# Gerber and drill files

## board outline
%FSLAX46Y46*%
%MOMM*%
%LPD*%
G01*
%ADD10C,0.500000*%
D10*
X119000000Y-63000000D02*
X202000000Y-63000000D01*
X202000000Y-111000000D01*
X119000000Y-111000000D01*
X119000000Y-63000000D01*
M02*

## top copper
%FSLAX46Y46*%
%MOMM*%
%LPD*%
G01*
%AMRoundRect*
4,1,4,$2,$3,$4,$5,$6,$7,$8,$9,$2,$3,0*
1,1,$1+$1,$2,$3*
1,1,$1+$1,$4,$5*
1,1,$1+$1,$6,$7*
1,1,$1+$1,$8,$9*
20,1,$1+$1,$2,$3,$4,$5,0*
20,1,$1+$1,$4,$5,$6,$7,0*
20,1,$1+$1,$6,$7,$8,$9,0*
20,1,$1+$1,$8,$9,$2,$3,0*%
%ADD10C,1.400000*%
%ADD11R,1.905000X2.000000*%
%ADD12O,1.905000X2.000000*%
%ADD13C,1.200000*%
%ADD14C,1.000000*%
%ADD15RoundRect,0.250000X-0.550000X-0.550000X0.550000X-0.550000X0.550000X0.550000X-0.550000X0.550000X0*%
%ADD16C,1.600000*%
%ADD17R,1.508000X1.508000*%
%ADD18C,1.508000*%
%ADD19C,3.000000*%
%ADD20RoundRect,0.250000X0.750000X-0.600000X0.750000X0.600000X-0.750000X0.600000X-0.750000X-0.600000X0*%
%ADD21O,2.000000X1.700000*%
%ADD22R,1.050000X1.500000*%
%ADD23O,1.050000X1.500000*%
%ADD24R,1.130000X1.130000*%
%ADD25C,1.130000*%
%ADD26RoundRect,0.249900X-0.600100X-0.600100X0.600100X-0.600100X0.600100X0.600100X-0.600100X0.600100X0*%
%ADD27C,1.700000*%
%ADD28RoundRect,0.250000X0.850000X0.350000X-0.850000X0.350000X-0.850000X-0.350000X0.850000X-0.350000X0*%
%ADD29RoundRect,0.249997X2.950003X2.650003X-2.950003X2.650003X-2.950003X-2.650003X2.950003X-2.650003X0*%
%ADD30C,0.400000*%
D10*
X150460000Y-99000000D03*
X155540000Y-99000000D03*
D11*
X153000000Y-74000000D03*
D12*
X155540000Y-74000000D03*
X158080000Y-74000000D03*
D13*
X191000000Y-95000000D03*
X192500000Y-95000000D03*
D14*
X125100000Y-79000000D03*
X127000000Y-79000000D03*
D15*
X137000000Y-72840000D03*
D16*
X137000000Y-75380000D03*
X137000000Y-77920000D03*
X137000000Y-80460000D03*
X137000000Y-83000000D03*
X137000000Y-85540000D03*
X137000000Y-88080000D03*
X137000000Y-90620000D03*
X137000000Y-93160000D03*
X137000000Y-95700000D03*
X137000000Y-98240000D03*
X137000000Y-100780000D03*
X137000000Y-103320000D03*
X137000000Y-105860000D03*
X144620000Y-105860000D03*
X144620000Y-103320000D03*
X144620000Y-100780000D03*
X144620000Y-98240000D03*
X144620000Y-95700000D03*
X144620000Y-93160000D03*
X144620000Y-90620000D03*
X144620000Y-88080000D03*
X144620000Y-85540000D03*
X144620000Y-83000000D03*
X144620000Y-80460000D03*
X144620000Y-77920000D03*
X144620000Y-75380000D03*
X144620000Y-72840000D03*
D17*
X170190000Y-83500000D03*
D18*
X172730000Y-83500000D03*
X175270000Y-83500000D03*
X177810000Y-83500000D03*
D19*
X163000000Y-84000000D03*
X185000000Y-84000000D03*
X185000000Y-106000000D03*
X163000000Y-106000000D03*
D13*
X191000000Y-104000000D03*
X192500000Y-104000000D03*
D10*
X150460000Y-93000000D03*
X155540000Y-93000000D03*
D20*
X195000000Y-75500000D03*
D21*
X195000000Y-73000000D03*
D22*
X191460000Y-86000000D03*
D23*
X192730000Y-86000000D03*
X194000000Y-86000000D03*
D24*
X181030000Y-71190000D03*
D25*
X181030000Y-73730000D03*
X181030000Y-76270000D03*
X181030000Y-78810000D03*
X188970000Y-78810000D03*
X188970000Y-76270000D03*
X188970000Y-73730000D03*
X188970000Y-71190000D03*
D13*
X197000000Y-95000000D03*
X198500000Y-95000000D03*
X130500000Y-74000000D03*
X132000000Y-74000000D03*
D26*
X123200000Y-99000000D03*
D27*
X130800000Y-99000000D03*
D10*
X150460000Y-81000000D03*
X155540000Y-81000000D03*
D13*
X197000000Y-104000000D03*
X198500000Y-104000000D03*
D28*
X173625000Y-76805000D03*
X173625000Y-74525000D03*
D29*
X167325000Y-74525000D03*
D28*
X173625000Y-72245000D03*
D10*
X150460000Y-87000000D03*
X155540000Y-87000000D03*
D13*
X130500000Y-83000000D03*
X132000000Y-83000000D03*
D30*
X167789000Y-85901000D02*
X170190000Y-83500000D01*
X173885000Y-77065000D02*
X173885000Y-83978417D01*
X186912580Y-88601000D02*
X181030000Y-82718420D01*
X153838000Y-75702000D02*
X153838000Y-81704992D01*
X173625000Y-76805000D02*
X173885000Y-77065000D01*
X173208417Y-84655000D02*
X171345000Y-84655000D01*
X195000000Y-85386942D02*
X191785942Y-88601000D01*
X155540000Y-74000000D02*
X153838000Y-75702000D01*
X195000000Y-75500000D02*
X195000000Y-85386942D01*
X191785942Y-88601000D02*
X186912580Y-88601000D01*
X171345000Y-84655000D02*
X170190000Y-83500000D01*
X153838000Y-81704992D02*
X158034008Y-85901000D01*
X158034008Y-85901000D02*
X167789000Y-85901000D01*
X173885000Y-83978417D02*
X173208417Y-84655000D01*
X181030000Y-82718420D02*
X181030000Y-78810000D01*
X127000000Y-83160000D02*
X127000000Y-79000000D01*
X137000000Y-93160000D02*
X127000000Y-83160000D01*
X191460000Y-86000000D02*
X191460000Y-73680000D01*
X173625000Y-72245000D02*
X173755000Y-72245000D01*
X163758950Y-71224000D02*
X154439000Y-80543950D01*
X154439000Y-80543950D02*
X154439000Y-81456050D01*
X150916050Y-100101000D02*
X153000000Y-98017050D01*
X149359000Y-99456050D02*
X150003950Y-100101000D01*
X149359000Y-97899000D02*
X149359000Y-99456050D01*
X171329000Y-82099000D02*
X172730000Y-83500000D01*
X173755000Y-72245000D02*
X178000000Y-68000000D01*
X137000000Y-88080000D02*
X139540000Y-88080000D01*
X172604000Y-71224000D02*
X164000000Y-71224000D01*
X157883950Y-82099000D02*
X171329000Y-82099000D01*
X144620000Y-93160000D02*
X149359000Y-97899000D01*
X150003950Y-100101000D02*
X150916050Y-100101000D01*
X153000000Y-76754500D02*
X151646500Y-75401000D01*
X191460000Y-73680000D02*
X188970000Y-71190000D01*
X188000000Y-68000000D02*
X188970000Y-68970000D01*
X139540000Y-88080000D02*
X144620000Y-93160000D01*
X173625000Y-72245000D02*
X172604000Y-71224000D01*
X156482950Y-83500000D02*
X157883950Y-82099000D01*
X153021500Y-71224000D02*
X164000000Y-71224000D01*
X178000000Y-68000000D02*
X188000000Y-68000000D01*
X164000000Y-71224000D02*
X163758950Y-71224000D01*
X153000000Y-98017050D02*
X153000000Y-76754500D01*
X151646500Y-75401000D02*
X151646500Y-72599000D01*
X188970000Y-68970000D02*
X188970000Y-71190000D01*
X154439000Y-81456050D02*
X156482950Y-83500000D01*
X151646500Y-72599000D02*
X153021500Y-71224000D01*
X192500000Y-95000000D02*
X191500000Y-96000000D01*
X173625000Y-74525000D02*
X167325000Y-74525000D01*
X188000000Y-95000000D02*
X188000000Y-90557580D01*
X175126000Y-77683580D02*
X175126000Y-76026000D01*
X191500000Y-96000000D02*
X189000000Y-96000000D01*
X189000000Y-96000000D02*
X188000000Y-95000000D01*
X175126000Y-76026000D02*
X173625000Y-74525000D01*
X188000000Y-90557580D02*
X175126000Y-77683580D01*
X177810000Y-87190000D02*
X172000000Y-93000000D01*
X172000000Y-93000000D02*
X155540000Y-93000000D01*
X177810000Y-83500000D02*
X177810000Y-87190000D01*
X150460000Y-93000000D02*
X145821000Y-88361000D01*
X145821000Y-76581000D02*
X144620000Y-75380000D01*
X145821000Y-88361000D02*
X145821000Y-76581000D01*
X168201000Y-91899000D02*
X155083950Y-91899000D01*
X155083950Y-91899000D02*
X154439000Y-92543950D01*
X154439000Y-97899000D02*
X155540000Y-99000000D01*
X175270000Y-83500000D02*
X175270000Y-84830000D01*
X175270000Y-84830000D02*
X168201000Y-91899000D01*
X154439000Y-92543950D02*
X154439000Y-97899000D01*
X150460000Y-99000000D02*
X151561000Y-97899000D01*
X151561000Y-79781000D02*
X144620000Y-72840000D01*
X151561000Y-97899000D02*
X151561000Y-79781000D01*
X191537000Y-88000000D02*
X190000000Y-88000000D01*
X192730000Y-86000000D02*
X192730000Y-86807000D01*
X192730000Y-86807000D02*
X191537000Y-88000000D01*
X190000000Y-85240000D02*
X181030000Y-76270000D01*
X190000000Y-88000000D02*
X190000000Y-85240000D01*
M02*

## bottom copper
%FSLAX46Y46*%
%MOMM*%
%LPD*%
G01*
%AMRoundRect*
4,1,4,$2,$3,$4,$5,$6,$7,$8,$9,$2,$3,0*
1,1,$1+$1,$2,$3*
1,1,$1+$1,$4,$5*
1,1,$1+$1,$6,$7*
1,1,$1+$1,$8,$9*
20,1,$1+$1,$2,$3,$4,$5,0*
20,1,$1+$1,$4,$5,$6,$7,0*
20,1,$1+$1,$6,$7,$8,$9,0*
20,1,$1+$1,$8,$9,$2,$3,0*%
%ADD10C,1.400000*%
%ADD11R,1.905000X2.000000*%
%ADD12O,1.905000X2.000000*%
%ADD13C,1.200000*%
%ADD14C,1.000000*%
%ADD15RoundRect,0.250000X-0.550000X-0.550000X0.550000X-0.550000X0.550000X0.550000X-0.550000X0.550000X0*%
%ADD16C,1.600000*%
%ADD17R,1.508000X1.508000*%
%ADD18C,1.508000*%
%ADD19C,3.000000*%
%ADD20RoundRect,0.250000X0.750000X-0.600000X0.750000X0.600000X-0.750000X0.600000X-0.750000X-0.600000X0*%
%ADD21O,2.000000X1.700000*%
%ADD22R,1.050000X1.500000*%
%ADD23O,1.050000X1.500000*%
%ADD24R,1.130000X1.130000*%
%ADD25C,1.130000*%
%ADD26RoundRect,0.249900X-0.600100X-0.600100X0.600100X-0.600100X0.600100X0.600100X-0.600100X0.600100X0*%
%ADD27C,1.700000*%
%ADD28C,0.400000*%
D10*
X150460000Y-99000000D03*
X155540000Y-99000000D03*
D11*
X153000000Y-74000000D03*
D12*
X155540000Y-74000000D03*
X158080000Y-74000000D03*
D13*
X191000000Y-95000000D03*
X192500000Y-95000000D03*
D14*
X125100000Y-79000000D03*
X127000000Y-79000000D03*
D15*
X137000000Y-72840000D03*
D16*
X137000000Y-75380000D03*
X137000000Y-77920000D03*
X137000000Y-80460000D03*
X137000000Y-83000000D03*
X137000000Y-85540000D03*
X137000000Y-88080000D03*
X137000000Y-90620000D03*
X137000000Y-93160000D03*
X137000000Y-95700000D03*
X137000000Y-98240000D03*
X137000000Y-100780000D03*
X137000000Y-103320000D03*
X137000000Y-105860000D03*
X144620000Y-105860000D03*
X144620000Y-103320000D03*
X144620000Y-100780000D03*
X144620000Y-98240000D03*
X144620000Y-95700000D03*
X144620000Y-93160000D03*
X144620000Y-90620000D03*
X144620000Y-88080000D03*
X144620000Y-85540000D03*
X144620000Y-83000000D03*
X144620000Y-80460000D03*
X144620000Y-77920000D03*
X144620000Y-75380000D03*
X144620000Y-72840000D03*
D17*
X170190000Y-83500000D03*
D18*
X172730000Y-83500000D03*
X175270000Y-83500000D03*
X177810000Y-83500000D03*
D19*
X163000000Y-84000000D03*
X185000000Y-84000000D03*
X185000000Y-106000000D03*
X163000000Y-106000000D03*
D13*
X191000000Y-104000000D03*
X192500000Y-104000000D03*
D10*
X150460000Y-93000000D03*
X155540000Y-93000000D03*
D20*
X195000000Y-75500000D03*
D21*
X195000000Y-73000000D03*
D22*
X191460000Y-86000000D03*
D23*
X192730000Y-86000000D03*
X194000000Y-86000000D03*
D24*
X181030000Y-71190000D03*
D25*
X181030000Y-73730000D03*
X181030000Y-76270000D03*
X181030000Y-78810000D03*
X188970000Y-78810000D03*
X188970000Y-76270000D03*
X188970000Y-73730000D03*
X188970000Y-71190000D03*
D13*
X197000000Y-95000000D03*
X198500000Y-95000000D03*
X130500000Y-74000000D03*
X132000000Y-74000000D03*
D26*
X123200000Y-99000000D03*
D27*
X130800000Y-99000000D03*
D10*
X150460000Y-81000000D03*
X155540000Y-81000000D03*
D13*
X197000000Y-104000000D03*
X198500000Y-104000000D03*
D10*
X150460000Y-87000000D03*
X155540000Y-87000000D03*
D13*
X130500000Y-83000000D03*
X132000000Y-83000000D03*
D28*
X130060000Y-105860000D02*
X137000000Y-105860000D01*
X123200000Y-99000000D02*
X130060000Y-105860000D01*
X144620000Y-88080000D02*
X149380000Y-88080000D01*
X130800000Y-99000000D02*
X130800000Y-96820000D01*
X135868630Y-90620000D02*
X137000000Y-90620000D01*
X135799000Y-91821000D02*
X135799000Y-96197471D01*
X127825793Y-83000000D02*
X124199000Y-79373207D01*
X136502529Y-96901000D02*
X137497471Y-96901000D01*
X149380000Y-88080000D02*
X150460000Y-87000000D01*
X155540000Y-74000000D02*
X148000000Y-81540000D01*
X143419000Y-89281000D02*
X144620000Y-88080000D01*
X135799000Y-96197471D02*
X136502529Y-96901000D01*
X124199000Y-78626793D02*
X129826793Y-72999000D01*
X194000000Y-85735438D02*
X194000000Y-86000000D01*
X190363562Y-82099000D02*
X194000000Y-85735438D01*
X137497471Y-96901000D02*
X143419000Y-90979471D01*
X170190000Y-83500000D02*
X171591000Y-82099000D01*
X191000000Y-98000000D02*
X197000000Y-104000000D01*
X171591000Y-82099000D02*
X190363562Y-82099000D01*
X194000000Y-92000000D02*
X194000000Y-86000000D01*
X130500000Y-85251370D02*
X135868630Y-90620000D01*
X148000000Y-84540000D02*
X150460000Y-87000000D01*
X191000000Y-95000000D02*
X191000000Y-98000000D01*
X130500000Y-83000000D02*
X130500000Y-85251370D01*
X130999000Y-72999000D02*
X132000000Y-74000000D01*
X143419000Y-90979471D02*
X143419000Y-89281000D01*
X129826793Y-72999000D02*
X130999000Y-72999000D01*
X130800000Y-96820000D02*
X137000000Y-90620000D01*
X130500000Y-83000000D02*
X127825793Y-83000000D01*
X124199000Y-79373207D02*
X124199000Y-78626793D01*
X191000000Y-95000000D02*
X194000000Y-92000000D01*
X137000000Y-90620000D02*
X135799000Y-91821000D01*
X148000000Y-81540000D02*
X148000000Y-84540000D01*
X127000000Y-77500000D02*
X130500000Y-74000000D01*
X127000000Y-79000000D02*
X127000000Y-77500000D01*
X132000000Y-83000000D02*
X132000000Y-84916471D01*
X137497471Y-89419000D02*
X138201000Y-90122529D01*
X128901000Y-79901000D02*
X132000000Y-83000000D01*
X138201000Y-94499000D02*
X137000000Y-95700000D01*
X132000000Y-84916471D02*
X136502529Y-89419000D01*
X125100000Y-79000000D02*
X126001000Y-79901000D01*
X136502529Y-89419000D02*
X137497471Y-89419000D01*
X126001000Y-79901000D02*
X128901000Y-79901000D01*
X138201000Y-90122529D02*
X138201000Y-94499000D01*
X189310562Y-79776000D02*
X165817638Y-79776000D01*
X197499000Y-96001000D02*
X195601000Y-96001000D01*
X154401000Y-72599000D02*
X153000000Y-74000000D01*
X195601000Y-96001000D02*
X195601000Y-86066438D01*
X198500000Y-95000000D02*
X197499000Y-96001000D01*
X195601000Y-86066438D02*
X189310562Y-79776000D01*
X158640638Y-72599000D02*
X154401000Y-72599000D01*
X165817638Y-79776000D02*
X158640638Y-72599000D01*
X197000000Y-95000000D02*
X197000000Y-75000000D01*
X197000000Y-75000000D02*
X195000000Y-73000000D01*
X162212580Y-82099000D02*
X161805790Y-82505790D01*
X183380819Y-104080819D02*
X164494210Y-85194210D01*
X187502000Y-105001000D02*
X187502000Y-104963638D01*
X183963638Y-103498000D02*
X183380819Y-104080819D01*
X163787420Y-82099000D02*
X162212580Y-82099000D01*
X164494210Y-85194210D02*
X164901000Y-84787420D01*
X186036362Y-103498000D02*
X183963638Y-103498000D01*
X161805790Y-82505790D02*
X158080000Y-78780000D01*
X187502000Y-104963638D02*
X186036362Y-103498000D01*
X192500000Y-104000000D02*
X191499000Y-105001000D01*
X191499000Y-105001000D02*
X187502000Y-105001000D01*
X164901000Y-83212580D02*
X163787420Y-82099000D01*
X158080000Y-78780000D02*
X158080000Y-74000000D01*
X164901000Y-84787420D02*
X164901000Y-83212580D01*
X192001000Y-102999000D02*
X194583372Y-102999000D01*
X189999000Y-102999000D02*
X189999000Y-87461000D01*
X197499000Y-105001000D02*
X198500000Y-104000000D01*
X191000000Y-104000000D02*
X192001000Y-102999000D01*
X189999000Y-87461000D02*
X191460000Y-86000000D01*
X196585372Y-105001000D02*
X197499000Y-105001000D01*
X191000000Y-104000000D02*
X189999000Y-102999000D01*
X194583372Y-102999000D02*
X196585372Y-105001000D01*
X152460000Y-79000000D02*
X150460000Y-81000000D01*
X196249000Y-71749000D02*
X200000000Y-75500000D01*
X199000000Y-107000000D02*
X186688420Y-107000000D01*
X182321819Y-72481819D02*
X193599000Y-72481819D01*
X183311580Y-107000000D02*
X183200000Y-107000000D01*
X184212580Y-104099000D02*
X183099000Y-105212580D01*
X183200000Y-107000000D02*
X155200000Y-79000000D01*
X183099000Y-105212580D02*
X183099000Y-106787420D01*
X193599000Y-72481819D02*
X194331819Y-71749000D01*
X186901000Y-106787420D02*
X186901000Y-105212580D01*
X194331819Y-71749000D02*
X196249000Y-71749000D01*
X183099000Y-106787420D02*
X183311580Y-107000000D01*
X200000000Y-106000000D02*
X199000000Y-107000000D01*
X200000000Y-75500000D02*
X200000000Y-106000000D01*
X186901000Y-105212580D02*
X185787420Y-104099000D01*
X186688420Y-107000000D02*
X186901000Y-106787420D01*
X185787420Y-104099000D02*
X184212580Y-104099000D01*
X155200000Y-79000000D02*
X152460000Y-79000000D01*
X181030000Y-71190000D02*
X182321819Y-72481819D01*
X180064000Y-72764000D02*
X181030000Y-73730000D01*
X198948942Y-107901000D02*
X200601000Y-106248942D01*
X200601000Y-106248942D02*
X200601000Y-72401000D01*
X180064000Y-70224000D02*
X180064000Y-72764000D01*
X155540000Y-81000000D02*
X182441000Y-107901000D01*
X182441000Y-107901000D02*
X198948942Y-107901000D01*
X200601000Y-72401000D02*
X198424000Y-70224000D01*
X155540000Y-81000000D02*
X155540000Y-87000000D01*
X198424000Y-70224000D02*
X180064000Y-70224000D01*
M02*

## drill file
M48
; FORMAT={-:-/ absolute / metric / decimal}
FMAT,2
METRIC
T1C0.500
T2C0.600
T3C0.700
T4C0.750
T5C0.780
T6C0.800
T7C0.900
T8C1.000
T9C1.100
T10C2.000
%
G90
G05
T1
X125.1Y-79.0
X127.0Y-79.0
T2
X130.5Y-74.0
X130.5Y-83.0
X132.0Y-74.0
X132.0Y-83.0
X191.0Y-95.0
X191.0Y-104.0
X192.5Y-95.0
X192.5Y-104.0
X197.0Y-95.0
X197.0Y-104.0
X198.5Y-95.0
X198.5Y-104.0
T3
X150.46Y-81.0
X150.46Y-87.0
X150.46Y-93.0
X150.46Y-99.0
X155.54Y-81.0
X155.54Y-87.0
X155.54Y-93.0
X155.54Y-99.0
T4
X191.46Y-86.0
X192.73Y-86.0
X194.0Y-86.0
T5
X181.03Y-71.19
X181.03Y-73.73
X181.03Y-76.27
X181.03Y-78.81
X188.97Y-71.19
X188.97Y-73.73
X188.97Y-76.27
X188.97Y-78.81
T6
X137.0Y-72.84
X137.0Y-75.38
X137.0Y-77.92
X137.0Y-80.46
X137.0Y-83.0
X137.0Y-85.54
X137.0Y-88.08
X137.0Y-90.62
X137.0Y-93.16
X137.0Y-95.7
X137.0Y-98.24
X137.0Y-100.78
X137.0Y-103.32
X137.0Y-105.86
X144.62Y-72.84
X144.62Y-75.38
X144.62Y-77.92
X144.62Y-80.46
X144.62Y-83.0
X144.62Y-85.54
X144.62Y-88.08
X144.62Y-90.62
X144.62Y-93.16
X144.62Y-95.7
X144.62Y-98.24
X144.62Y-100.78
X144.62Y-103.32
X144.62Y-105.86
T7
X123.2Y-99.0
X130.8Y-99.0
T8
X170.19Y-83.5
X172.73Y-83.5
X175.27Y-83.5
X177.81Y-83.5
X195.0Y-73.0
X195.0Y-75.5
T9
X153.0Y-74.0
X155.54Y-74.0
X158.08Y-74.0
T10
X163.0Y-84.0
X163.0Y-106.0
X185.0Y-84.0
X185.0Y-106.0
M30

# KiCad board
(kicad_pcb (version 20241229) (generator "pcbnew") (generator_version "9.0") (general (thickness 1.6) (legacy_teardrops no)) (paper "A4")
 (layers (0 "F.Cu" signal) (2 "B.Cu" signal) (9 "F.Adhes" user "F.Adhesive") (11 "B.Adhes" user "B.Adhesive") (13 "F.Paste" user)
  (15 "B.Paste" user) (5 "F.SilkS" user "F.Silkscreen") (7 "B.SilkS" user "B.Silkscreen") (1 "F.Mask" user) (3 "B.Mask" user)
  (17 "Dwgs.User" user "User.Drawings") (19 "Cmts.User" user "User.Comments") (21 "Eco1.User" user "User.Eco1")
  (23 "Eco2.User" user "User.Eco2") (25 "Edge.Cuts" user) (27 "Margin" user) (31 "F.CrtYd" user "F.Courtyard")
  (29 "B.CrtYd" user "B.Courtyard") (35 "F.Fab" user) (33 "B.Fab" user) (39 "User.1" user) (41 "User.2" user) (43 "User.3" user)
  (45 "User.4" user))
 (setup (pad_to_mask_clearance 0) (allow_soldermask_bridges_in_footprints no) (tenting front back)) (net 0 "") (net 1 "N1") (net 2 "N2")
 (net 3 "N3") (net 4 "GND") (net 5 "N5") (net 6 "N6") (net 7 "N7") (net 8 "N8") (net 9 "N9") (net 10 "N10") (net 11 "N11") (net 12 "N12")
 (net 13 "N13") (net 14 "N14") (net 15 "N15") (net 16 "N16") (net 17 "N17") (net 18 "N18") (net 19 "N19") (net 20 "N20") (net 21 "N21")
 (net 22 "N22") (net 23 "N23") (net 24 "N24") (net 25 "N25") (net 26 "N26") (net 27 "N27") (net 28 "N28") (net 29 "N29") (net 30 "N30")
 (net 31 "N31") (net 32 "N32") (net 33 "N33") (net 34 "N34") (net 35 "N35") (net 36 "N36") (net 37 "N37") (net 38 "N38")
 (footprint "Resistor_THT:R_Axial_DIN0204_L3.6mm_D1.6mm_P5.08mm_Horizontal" (layer "F.Cu") (at 150.46 99)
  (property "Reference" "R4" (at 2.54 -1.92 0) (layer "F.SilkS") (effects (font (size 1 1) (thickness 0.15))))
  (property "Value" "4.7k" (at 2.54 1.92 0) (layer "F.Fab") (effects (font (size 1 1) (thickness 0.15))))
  (pad "1" thru_hole circle (at 0 0) (size 1.4 1.4) (drill 0.7) (layers "*.Cu" "*.Mask") (remove_unused_layers no) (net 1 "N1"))
  (pad "2" thru_hole circle (at 5.08 0) (size 1.4 1.4) (drill 0.7) (layers "*.Cu" "*.Mask") (remove_unused_layers no) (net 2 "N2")))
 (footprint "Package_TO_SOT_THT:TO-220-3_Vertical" (layer "F.Cu") (at 153 74)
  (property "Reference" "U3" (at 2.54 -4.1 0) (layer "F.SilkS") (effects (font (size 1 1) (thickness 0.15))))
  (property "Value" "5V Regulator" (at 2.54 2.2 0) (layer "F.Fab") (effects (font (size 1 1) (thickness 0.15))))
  (pad "1" thru_hole rect (at 0 0) (size 1.905 2) (drill 1.1) (layers "*.Cu" "*.Mask") (remove_unused_layers no) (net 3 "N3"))
  (pad "2" thru_hole oval (at 2.54 0) (size 1.905 2) (drill 1.1) (layers "*.Cu" "*.Mask") (remove_unused_layers no) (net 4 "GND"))
  (pad "3" thru_hole oval (at 5.08 0) (size 1.905 2) (drill 1.1) (layers "*.Cu" "*.Mask") (remove_unused_layers no) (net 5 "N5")))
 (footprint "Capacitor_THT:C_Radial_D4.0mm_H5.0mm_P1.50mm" (layer "F.Cu") (at 191 95)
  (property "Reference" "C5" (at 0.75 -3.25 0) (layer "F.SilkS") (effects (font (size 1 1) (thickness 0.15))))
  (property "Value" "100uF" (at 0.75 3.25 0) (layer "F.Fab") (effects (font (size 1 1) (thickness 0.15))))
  (pad "1" thru_hole circle (at 0 0) (size 1.2 1.2) (drill 0.6) (layers "*.Cu" "*.Mask") (remove_unused_layers no) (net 4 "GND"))
  (pad "2" thru_hole circle (at 1.5 0) (size 1.2 1.2) (drill 0.6) (layers "*.Cu" "*.Mask") (remove_unused_layers no) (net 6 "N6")))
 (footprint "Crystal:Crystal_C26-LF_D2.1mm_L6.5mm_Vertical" (layer "F.Cu") (at 125.1 79)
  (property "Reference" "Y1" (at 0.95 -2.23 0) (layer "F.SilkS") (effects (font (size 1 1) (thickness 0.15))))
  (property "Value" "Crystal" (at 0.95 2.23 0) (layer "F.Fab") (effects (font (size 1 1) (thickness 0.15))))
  (pad "1" thru_hole circle (at 0 0) (size 1 1) (drill 0.5) (layers "*.Cu" "*.Mask") (remove_unused_layers no) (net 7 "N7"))
  (pad "2" thru_hole circle (at 1.9 0) (size 1 1) (drill 0.5) (layers "*.Cu" "*.Mask") (remove_unused_layers no) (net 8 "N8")))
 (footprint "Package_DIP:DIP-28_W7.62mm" (layer "F.Cu") (at 137 72.84)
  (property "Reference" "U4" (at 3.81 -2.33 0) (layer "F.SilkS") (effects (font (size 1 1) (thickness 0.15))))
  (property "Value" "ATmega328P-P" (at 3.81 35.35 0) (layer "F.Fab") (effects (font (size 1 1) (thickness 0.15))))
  (pad "1" thru_hole roundrect (at 0 0) (size 1.6 1.6) (drill 0.8) (layers "*.Cu" "*.Mask") (remove_unused_layers no)
   (roundrect_rratio 0.15625) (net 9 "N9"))
  (pad "2" thru_hole circle (at 0 2.54) (size 1.6 1.6) (drill 0.8) (layers "*.Cu" "*.Mask") (remove_unused_layers no) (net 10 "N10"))
  (pad "3" thru_hole circle (at 0 5.08) (size 1.6 1.6) (drill 0.8) (layers "*.Cu" "*.Mask") (remove_unused_layers no) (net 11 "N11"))
  (pad "4" thru_hole circle (at 0 7.62) (size 1.6 1.6) (drill 0.8) (layers "*.Cu" "*.Mask") (remove_unused_layers no) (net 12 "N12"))
  (pad "5" thru_hole circle (at 0 10.16) (size 1.6 1.6) (drill 0.8) (layers "*.Cu" "*.Mask") (remove_unused_layers no) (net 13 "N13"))
  (pad "6" thru_hole circle (at 0 12.7) (size 1.6 1.6) (drill 0.8) (layers "*.Cu" "*.Mask") (remove_unused_layers no) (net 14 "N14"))
  (pad "7" thru_hole circle (at 0 15.24) (size 1.6 1.6) (drill 0.8) (layers "*.Cu" "*.Mask") (remove_unused_layers no) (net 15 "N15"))
  (pad "8" thru_hole circle (at 0 17.78) (size 1.6 1.6) (drill 0.8) (layers "*.Cu" "*.Mask") (remove_unused_layers no) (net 4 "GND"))
  (pad "9" thru_hole circle (at 0 20.32) (size 1.6 1.6) (drill 0.8) (layers "*.Cu" "*.Mask") (remove_unused_layers no) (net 8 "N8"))
  (pad "10" thru_hole circle (at 0 22.86) (size 1.6 1.6) (drill 0.8) (layers "*.Cu" "*.Mask") (remove_unused_layers no) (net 7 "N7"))
  (pad "11" thru_hole circle (at 0 25.4) (size 1.6 1.6) (drill 0.8) (layers "*.Cu" "*.Mask") (remove_unused_layers no) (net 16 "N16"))
  (pad "12" thru_hole circle (at 0 27.94) (size 1.6 1.6) (drill 0.8) (layers "*.Cu" "*.Mask") (remove_unused_layers no) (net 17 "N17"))
  (pad "13" thru_hole circle (at 0 30.48) (size 1.6 1.6) (drill 0.8) (layers "*.Cu" "*.Mask") (remove_unused_layers no) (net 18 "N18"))
  (pad "14" thru_hole circle (at 0 33.02) (size 1.6 1.6) (drill 0.8) (layers "*.Cu" "*.Mask") (remove_unused_layers no) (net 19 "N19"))
  (pad "15" thru_hole circle (at 7.62 33.02) (size 1.6 1.6) (drill 0.8) (layers "*.Cu" "*.Mask") (remove_unused_layers no) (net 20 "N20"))
  (pad "16" thru_hole circle (at 7.62 30.48) (size 1.6 1.6) (drill 0.8) (layers "*.Cu" "*.Mask") (remove_unused_layers no) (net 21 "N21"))
  (pad "17" thru_hole circle (at 7.62 27.94) (size 1.6 1.6) (drill 0.8) (layers "*.Cu" "*.Mask") (remove_unused_layers no) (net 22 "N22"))
  (pad "18" thru_hole circle (at 7.62 25.4) (size 1.6 1.6) (drill 0.8) (layers "*.Cu" "*.Mask") (remove_unused_layers no) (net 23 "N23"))
  (pad "19" thru_hole circle (at 7.62 22.86) (size 1.6 1.6) (drill 0.8) (layers "*.Cu" "*.Mask") (remove_unused_layers no) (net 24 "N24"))
  (pad "20" thru_hole circle (at 7.62 20.32) (size 1.6 1.6) (drill 0.8) (layers "*.Cu" "*.Mask") (remove_unused_layers no) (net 15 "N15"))
  (pad "21" thru_hole circle (at 7.62 17.78) (size 1.6 1.6) (drill 0.8) (layers "*.Cu" "*.Mask") (remove_unused_layers no) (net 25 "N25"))
  (pad "22" thru_hole circle (at 7.62 15.24) (size 1.6 1.6) (drill 0.8) (layers "*.Cu" "*.Mask") (remove_unused_layers no) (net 4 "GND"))
  (pad "23" thru_hole circle (at 7.62 12.7) (size 1.6 1.6) (drill 0.8) (layers "*.Cu" "*.Mask") (remove_unused_layers no) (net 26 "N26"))
  (pad "24" thru_hole circle (at 7.62 10.16) (size 1.6 1.6) (drill 0.8) (layers "*.Cu" "*.Mask") (remove_unused_layers no) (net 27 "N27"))
  (pad "25" thru_hole circle (at 7.62 7.62) (size 1.6 1.6) (drill 0.8) (layers "*.Cu" "*.Mask") (remove_unused_layers no) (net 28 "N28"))
  (pad "26" thru_hole circle (at 7.62 5.08) (size 1.6 1.6) (drill 0.8) (layers "*.Cu" "*.Mask") (remove_unused_layers no) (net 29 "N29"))
  (pad "27" thru_hole circle (at 7.62 2.54) (size 1.6 1.6) (drill 0.8) (layers "*.Cu" "*.Mask") (remove_unused_layers no) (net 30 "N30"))
  (pad "28" thru_hole circle (at 7.62 0) (size 1.6 1.6) (drill 0.8) (layers "*.Cu" "*.Mask") (remove_unused_layers no) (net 1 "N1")))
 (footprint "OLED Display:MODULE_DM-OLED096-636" (layer "F.Cu") (at 174 95)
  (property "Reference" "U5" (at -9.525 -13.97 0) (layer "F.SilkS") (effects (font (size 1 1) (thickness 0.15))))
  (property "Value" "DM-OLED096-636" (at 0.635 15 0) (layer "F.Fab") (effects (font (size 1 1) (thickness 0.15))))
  (pad "1" thru_hole rect (at -3.81 -11.5) (size 1.508 1.508) (drill 1) (layers "*.Cu" "*.Mask") (remove_unused_layers no) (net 4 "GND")
   (solder_mask_margin 0.102))
  (pad "2" thru_hole circle (at -1.27 -11.5) (size 1.508 1.508) (drill 1) (layers "*.Cu" "*.Mask") (remove_unused_layers no) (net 15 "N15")
   (solder_mask_margin 0.102))
  (pad "3" thru_hole circle (at 1.27 -11.5) (size 1.508 1.508) (drill 1) (layers "*.Cu" "*.Mask") (remove_unused_layers no) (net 2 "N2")
   (solder_mask_margin 0.102))
  (pad "4" thru_hole circle (at 3.81 -11.5) (size 1.508 1.508) (drill 1) (layers "*.Cu" "*.Mask") (remove_unused_layers no) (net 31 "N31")
   (solder_mask_margin 0.102))
  (pad "S1" thru_hole circle (at -11 -11) (size 3 3) (drill 2) (layers "*.Cu" "*.Mask") (remove_unused_layers no) (solder_mask_margin 0.102))
  (pad "S2" thru_hole circle (at 11 -11) (size 3 3) (drill 2) (layers "*.Cu" "*.Mask") (remove_unused_layers no) (solder_mask_margin 0.102))
  (pad "S3" thru_hole circle (at 11 11) (size 3 3) (drill 2) (layers "*.Cu" "*.Mask") (remove_unused_layers no) (solder_mask_margin 0.102))
  (pad "S4" thru_hole circle (at -11 11) (size 3 3) (drill 2) (layers "*.Cu" "*.Mask") (remove_unused_layers no) (solder_mask_margin 0.102)))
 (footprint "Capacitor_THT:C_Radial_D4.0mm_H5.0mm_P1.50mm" (layer "F.Cu") (at 191 104)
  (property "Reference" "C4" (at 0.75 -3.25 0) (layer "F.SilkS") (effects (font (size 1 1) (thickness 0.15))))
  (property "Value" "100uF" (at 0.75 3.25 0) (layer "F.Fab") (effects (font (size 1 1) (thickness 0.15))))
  (pad "1" thru_hole circle (at 0 0) (size 1.2 1.2) (drill 0.6) (layers "*.Cu" "*.Mask") (remove_unused_layers no) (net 15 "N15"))
  (pad "2" thru_hole circle (at 1.5 0) (size 1.2 1.2) (drill 0.6) (layers "*.Cu" "*.Mask") (remove_unused_layers no) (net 5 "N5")))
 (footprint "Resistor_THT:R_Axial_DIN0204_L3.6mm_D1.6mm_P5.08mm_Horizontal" (layer "F.Cu") (at 150.46 93)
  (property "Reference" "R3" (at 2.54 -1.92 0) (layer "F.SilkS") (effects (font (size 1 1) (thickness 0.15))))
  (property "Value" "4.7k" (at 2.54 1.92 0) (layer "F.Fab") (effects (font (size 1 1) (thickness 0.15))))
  (pad "1" thru_hole circle (at 0 0) (size 1.4 1.4) (drill 0.7) (layers "*.Cu" "*.Mask") (remove_unused_layers no) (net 30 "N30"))
  (pad "2" thru_hole circle (at 5.08 0) (size 1.4 1.4) (drill 0.7) (layers "*.Cu" "*.Mask") (remove_unused_layers no) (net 31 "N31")))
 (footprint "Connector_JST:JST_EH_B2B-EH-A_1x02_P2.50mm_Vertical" (layer "F.Cu") (at 195 75.5 90)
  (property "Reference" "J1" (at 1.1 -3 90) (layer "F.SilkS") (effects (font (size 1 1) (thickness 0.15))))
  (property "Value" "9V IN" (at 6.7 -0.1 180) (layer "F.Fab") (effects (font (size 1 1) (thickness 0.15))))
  (pad "1" thru_hole roundrect (at 0 0 90) (size 1.7 2) (drill 1) (layers "*.Cu" "*.Mask") (remove_unused_layers no)
   (roundrect_rratio 0.147059) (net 4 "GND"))
  (pad "2" thru_hole oval (at 2.5 0 90) (size 1.7 2) (drill 1) (layers "*.Cu" "*.Mask") (remove_unused_layers no) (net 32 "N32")))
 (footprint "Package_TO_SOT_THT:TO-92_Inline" (layer "F.Cu") (at 191.46 86)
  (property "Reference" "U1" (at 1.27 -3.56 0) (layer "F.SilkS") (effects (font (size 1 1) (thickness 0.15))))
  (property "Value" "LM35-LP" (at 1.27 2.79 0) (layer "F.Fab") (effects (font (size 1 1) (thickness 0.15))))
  (pad "1" thru_hole rect (at 0 0) (size 1.05 1.5) (drill 0.75) (layers "*.Cu" "*.Mask") (remove_unused_layers no) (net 15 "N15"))
  (pad "2" thru_hole oval (at 1.27 0) (size 1.05 1.5) (drill 0.75) (layers "*.Cu" "*.Mask") (remove_unused_layers no) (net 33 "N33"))
  (pad "3" thru_hole oval (at 2.54 0) (size 1.05 1.5) (drill 0.75) (layers "*.Cu" "*.Mask") (remove_unused_layers no) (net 4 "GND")))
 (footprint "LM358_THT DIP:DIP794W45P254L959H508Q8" (layer "F.Cu") (at 185 75)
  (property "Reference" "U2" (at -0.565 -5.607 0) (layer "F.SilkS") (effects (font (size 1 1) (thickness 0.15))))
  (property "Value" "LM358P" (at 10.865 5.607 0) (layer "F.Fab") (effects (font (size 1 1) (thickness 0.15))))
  (pad "1" thru_hole rect (at -3.97 -3.81) (size 1.13 1.13) (drill 0.78) (layers "*.Cu" "*.Mask") (remove_unused_layers no) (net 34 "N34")
   (solder_mask_margin 0.102))
  (pad "2" thru_hole circle (at -3.97 -1.27) (size 1.13 1.13) (drill 0.78) (layers "*.Cu" "*.Mask") (remove_unused_layers no) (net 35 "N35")
   (solder_mask_margin 0.102))
  (pad "3" thru_hole circle (at -3.97 1.27) (size 1.13 1.13) (drill 0.78) (layers "*.Cu" "*.Mask") (remove_unused_layers no) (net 33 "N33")
   (solder_mask_margin 0.102))
  (pad "4" thru_hole circle (at -3.97 3.81) (size 1.13 1.13) (drill 0.78) (layers "*.Cu" "*.Mask") (remove_unused_layers no) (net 4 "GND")
   (solder_mask_margin 0.102))
  (pad "5" thru_hole circle (at 3.97 3.81) (size 1.13 1.13) (drill 0.78) (layers "*.Cu" "*.Mask") (remove_unused_layers no) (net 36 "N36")
   (solder_mask_margin 0.102))
  (pad "6" thru_hole circle (at 3.97 1.27) (size 1.13 1.13) (drill 0.78) (layers "*.Cu" "*.Mask") (remove_unused_layers no) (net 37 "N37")
   (solder_mask_margin 0.102))
  (pad "7" thru_hole circle (at 3.97 -1.27) (size 1.13 1.13) (drill 0.78) (layers "*.Cu" "*.Mask") (remove_unused_layers no) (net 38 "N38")
   (solder_mask_margin 0.102))
  (pad "8" thru_hole circle (at 3.97 -3.81) (size 1.13 1.13) (drill 0.78) (layers "*.Cu" "*.Mask") (remove_unused_layers no) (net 15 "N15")
   (solder_mask_margin 0.102)))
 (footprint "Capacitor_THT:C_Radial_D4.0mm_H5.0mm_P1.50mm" (layer "F.Cu") (at 197 95)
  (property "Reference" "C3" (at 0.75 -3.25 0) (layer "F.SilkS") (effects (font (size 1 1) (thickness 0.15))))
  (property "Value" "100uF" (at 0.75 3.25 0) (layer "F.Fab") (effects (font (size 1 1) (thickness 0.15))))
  (pad "1" thru_hole circle (at 0 0) (size 1.2 1.2) (drill 0.6) (layers "*.Cu" "*.Mask") (remove_unused_layers no) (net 32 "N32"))
  (pad "2" thru_hole circle (at 1.5 0) (size 1.2 1.2) (drill 0.6) (layers "*.Cu" "*.Mask") (remove_unused_layers no) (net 3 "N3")))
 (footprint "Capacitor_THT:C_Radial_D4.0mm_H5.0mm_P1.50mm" (layer "F.Cu") (at 130.5 74)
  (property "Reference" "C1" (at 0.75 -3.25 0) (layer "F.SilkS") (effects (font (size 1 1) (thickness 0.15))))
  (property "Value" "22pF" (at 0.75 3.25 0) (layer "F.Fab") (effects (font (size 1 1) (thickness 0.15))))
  (pad "1" thru_hole circle (at 0 0) (size 1.2 1.2) (drill 0.6) (layers "*.Cu" "*.Mask") (remove_unused_layers no) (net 8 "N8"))
  (pad "2" thru_hole circle (at 1.5 0) (size 1.2 1.2) (drill 0.6) (layers "*.Cu" "*.Mask") (remove_unused_layers no) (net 4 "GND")))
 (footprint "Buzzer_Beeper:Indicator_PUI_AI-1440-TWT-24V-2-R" (layer "F.Cu") (at 123.2 99)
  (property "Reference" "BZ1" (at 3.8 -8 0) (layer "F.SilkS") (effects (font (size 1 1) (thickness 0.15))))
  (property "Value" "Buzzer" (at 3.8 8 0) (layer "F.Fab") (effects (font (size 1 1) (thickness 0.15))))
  (pad "1" thru_hole roundrect (at 0 0) (size 1.7 1.7) (drill 0.9) (layers "*.Cu" "*.Mask") (remove_unused_layers no)
   (roundrect_rratio 0.147) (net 19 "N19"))
  (pad "2" thru_hole circle (at 7.6 0) (size 1.7 1.7) (drill 0.9) (layers "*.Cu" "*.Mask") (remove_unused_layers no) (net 4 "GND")))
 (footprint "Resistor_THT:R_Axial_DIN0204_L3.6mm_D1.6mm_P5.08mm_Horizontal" (layer "F.Cu") (at 150.46 81)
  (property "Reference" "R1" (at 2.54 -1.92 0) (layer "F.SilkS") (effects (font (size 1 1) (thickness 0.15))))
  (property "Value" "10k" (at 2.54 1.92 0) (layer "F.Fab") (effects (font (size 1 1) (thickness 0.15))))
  (pad "1" thru_hole circle (at 0 0) (size 1.4 1.4) (drill 0.7) (layers "*.Cu" "*.Mask") (remove_unused_layers no) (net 34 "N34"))
  (pad "2" thru_hole circle (at 5.08 0) (size 1.4 1.4) (drill 0.7) (layers "*.Cu" "*.Mask") (remove_unused_layers no) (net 35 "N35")))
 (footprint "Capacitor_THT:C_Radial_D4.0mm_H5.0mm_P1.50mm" (layer "F.Cu") (at 197 104)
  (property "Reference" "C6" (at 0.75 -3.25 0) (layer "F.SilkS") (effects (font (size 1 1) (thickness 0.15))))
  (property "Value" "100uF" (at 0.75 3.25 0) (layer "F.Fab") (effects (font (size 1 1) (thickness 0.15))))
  (pad "1" thru_hole circle (at 0 0) (size 1.2 1.2) (drill 0.6) (layers "*.Cu" "*.Mask") (remove_unused_layers no) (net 4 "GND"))
  (pad "2" thru_hole circle (at 1.5 0) (size 1.2 1.2) (drill 0.6) (layers "*.Cu" "*.Mask") (remove_unused_layers no) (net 15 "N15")))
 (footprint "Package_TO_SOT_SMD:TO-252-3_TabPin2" (layer "F.Cu") (at 168.585 74.525 180)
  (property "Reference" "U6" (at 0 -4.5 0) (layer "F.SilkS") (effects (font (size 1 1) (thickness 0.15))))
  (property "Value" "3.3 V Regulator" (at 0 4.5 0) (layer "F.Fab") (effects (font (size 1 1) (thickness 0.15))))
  (pad "" smd roundrect (at -0.415 -1.525 180) (size 3.05 2.75) (layers "F.Paste") (roundrect_rratio 0.090909))
  (pad "" smd roundrect (at -0.415 1.525 180) (size 3.05 2.75) (layers "F.Paste") (roundrect_rratio 0.090909))
  (pad "" smd roundrect (at 2.935 -1.525 180) (size 3.05 2.75) (layers "F.Paste") (roundrect_rratio 0.090909))
  (pad "" smd roundrect (at 2.935 1.525 180) (size 3.05 2.75) (layers "F.Paste") (roundrect_rratio 0.090909))
  (pad "1" smd roundrect (at -5.04 -2.28 180) (size 2.2 1.2) (layers "F.Cu" "F.Mask" "F.Paste") (roundrect_rratio 0.208333) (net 4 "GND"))
  (pad "2" smd roundrect (at -5.04 0 180) (size 2.2 1.2) (layers "F.Cu" "F.Mask" "F.Paste") (roundrect_rratio 0.208333) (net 6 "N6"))
  (pad "2" smd roundrect (at 1.26 0 180) (size 6.4 5.8) (layers "F.Cu" "F.Mask") (roundrect_rratio 0.043103) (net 6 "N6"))
  (pad "3" smd roundrect (at -5.04 2.28 180) (size 2.2 1.2) (layers "F.Cu" "F.Mask" "F.Paste") (roundrect_rratio 0.208333) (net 15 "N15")))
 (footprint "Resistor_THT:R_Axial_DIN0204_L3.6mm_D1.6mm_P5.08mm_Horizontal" (layer "F.Cu") (at 150.46 87)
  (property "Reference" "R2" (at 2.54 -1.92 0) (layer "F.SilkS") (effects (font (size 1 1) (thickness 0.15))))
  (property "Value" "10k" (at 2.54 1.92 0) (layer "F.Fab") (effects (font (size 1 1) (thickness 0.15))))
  (pad "1" thru_hole circle (at 0 0) (size 1.4 1.4) (drill 0.7) (layers "*.Cu" "*.Mask") (remove_unused_layers no) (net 4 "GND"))
  (pad "2" thru_hole circle (at 5.08 0) (size 1.4 1.4) (drill 0.7) (layers "*.Cu" "*.Mask") (remove_unused_layers no) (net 35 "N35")))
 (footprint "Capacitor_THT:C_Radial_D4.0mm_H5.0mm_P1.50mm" (layer "F.Cu") (at 130.5 83)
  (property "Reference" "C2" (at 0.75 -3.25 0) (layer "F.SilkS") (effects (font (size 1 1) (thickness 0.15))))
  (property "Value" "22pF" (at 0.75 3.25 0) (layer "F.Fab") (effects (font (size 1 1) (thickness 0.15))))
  (pad "1" thru_hole circle (at 0 0) (size 1.2 1.2) (drill 0.6) (layers "*.Cu" "*.Mask") (remove_unused_layers no) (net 4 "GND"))
  (pad "2" thru_hole circle (at 1.5 0) (size 1.2 1.2) (drill 0.6) (layers "*.Cu" "*.Mask") (remove_unused_layers no) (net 7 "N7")))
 (gr_rect (start 119 63) (end 202 111) (stroke (width 0.5) (type solid)) (fill no) (layer "Edge.Cuts"))
 (segment (start 130.06 105.86) (end 137 105.86) (width 0.4) (layer "B.Cu") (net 19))
 (segment (start 123.2 99) (end 130.06 105.86) (width 0.4) (layer "B.Cu") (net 19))
 (segment (start 167.789 85.901) (end 170.19 83.5) (width 0.4) (layer "F.Cu") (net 4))
 (segment (start 173.885 77.065) (end 173.885 83.978417) (width 0.4) (layer "F.Cu") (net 4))
 (segment (start 186.91258 88.601) (end 181.03 82.71842) (width 0.4) (layer "F.Cu") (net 4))
 (segment (start 153.838 75.702) (end 153.838 81.704992) (width 0.4) (layer "F.Cu") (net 4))
 (segment (start 173.625 76.805) (end 173.885 77.065) (width 0.4) (layer "F.Cu") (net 4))
 (segment (start 173.208417 84.655) (end 171.345 84.655) (width 0.4) (layer "F.Cu") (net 4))
 (segment (start 195 85.386942) (end 191.785942 88.601) (width 0.4) (layer "F.Cu") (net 4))
 (segment (start 155.54 74) (end 153.838 75.702) (width 0.4) (layer "F.Cu") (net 4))
 (segment (start 195 75.5) (end 195 85.386942) (width 0.4) (layer "F.Cu") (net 4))
 (segment (start 191.785942 88.601) (end 186.91258 88.601) (width 0.4) (layer "F.Cu") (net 4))
 (segment (start 171.345 84.655) (end 170.19 83.5) (width 0.4) (layer "F.Cu") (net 4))
 (segment (start 153.838 81.704992) (end 158.034008 85.901) (width 0.4) (layer "F.Cu") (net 4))
 (segment (start 158.034008 85.901) (end 167.789 85.901) (width 0.4) (layer "F.Cu") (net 4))
 (segment (start 173.885 83.978417) (end 173.208417 84.655) (width 0.4) (layer "F.Cu") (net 4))
 (segment (start 181.03 82.71842) (end 181.03 78.81) (width 0.4) (layer "F.Cu") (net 4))
 (segment (start 144.62 88.08) (end 149.38 88.08) (width 0.4) (layer "B.Cu") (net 4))
 (segment (start 130.8 99) (end 130.8 96.82) (width 0.4) (layer "B.Cu") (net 4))
 (segment (start 135.86863 90.62) (end 137 90.62) (width 0.4) (layer "B.Cu") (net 4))
 (segment (start 135.799 91.821) (end 135.799 96.197471) (width 0.4) (layer "B.Cu") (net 4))
 (segment (start 127.825793 83) (end 124.199 79.373207) (width 0.4) (layer "B.Cu") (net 4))
 (segment (start 136.502529 96.901) (end 137.497471 96.901) (width 0.4) (layer "B.Cu") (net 4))
 (segment (start 149.38 88.08) (end 150.46 87) (width 0.4) (layer "B.Cu") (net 4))
 (segment (start 155.54 74) (end 148 81.54) (width 0.4) (layer "B.Cu") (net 4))
 (segment (start 143.419 89.281) (end 144.62 88.08) (width 0.4) (layer "B.Cu") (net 4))
 (segment (start 135.799 96.197471) (end 136.502529 96.901) (width 0.4) (layer "B.Cu") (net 4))
 (segment (start 124.199 78.626793) (end 129.826793 72.999) (width 0.4) (layer "B.Cu") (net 4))
 (segment (start 194 85.735438) (end 194 86) (width 0.4) (layer "B.Cu") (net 4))
 (segment (start 190.363562 82.099) (end 194 85.735438) (width 0.4) (layer "B.Cu") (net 4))
 (segment (start 137.497471 96.901) (end 143.419 90.979471) (width 0.4) (layer "B.Cu") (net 4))
 (segment (start 170.19 83.5) (end 171.591 82.099) (width 0.4) (layer "B.Cu") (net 4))
 (segment (start 191 98) (end 197 104) (width 0.4) (layer "B.Cu") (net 4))
 (segment (start 171.591 82.099) (end 190.363562 82.099) (width 0.4) (layer "B.Cu") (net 4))
 (segment (start 194 92) (end 194 86) (width 0.4) (layer "B.Cu") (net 4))
 (segment (start 130.5 85.25137) (end 135.86863 90.62) (width 0.4) (layer "B.Cu") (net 4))
 (segment (start 148 84.54) (end 150.46 87) (width 0.4) (layer "B.Cu") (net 4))
 (segment (start 191 95) (end 191 98) (width 0.4) (layer "B.Cu") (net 4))
 (segment (start 130.5 83) (end 130.5 85.25137) (width 0.4) (layer "B.Cu") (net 4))
 (segment (start 130.999 72.999) (end 132 74) (width 0.4) (layer "B.Cu") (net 4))
 (segment (start 143.419 90.979471) (end 143.419 89.281) (width 0.4) (layer "B.Cu") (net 4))
 (segment (start 129.826793 72.999) (end 130.999 72.999) (width 0.4) (layer "B.Cu") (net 4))
 (segment (start 130.8 96.82) (end 137 90.62) (width 0.4) (layer "B.Cu") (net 4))
 (segment (start 130.5 83) (end 127.825793 83) (width 0.4) (layer "B.Cu") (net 4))
 (segment (start 124.199 79.373207) (end 124.199 78.626793) (width 0.4) (layer "B.Cu") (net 4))
 (segment (start 191 95) (end 194 92) (width 0.4) (layer "B.Cu") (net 4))
 (segment (start 137 90.62) (end 135.799 91.821) (width 0.4) (layer "B.Cu") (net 4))
 (segment (start 148 81.54) (end 148 84.54) (width 0.4) (layer "B.Cu") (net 4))
 (segment (start 127 83.16) (end 127 79) (width 0.4) (layer "F.Cu") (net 8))
 (segment (start 137 93.16) (end 127 83.16) (width 0.4) (layer "F.Cu") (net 8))
 (segment (start 127 77.5) (end 130.5 74) (width 0.4) (layer "B.Cu") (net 8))
 (segment (start 127 79) (end 127 77.5) (width 0.4) (layer "B.Cu") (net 8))
 (segment (start 132 83) (end 132 84.916471) (width 0.4) (layer "B.Cu") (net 7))
 (segment (start 137.497471 89.419) (end 138.201 90.122529) (width 0.4) (layer "B.Cu") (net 7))
 (segment (start 128.901 79.901) (end 132 83) (width 0.4) (layer "B.Cu") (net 7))
 (segment (start 138.201 94.499) (end 137 95.7) (width 0.4) (layer "B.Cu") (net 7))
 (segment (start 132 84.916471) (end 136.502529 89.419) (width 0.4) (layer "B.Cu") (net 7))
 (segment (start 125.1 79) (end 126.001 79.901) (width 0.4) (layer "B.Cu") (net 7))
 (segment (start 136.502529 89.419) (end 137.497471 89.419) (width 0.4) (layer "B.Cu") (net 7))
 (segment (start 126.001 79.901) (end 128.901 79.901) (width 0.4) (layer "B.Cu") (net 7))
 (segment (start 138.201 90.122529) (end 138.201 94.499) (width 0.4) (layer "B.Cu") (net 7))
 (segment (start 189.310562 79.776) (end 165.817638 79.776) (width 0.4) (layer "B.Cu") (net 3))
 (segment (start 197.499 96.001) (end 195.601 96.001) (width 0.4) (layer "B.Cu") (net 3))
 (segment (start 154.401 72.599) (end 153 74) (width 0.4) (layer "B.Cu") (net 3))
 (segment (start 195.601 96.001) (end 195.601 86.066438) (width 0.4) (layer "B.Cu") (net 3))
 (segment (start 198.5 95) (end 197.499 96.001) (width 0.4) (layer "B.Cu") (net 3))
 (segment (start 195.601 86.066438) (end 189.310562 79.776) (width 0.4) (layer "B.Cu") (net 3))
 (segment (start 158.640638 72.599) (end 154.401 72.599) (width 0.4) (layer "B.Cu") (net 3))
 (segment (start 165.817638 79.776) (end 158.640638 72.599) (width 0.4) (layer "B.Cu") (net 3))
 (segment (start 197 95) (end 197 75) (width 0.4) (layer "B.Cu") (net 32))
 (segment (start 197 75) (end 195 73) (width 0.4) (layer "B.Cu") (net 32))
 (segment (start 162.21258 82.099) (end 161.80579 82.50579) (width 0.4) (layer "B.Cu") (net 5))
 (segment (start 183.380819 104.080819) (end 164.49421 85.19421) (width 0.4) (layer "B.Cu") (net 5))
 (segment (start 187.502 105.001) (end 187.502 104.963638) (width 0.4) (layer "B.Cu") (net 5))
 (segment (start 183.963638 103.498) (end 183.380819 104.080819) (width 0.4) (layer "B.Cu") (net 5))
 (segment (start 163.78742 82.099) (end 162.21258 82.099) (width 0.4) (layer "B.Cu") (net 5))
 (segment (start 164.49421 85.19421) (end 164.901 84.78742) (width 0.4) (layer "B.Cu") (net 5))
 (segment (start 186.036362 103.498) (end 183.963638 103.498) (width 0.4) (layer "B.Cu") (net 5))
 (segment (start 161.80579 82.50579) (end 158.08 78.78) (width 0.4) (layer "B.Cu") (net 5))
 (segment (start 187.502 104.963638) (end 186.036362 103.498) (width 0.4) (layer "B.Cu") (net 5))
 (segment (start 192.5 104) (end 191.499 105.001) (width 0.4) (layer "B.Cu") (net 5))
 (segment (start 191.499 105.001) (end 187.502 105.001) (width 0.4) (layer "B.Cu") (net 5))
 (segment (start 164.901 83.21258) (end 163.78742 82.099) (width 0.4) (layer "B.Cu") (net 5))
 (segment (start 158.08 78.78) (end 158.08 74) (width 0.4) (layer "B.Cu") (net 5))
 (segment (start 164.901 84.78742) (end 164.901 83.21258) (width 0.4) (layer "B.Cu") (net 5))
 (segment (start 191.46 86) (end 191.46 73.68) (width 0.4) (layer "F.Cu") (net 15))
 (segment (start 173.625 72.245) (end 173.755 72.245) (width 0.4) (layer "F.Cu") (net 15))
 (segment (start 163.75895 71.224) (end 154.439 80.54395) (width 0.4) (layer "F.Cu") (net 15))
 (segment (start 154.439 80.54395) (end 154.439 81.45605) (width 0.4) (layer "F.Cu") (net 15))
 (segment (start 150.91605 100.101) (end 153 98.01705) (width 0.4) (layer "F.Cu") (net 15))
 (segment (start 149.359 99.45605) (end 150.00395 100.101) (width 0.4) (layer "F.Cu") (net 15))
 (segment (start 149.359 97.899) (end 149.359 99.45605) (width 0.4) (layer "F.Cu") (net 15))
 (segment (start 171.329 82.099) (end 172.73 83.5) (width 0.4) (layer "F.Cu") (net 15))
 (segment (start 173.755 72.245) (end 178 68) (width 0.4) (layer "F.Cu") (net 15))
 (segment (start 137 88.08) (end 139.54 88.08) (width 0.4) (layer "F.Cu") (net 15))
 (segment (start 172.604 71.224) (end 164 71.224) (width 0.4) (layer "F.Cu") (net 15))
 (segment (start 157.88395 82.099) (end 171.329 82.099) (width 0.4) (layer "F.Cu") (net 15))
 (segment (start 144.62 93.16) (end 149.359 97.899) (width 0.4) (layer "F.Cu") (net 15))
 (segment (start 150.00395 100.101) (end 150.91605 100.101) (width 0.4) (layer "F.Cu") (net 15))
 (segment (start 153 76.7545) (end 151.6465 75.401) (width 0.4) (layer "F.Cu") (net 15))
 (segment (start 191.46 73.68) (end 188.97 71.19) (width 0.4) (layer "F.Cu") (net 15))
 (segment (start 188 68) (end 188.97 68.97) (width 0.4) (layer "F.Cu") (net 15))
 (segment (start 139.54 88.08) (end 144.62 93.16) (width 0.4) (layer "F.Cu") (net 15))
 (segment (start 173.625 72.245) (end 172.604 71.224) (width 0.4) (layer "F.Cu") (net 15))
 (segment (start 156.48295 83.5) (end 157.88395 82.099) (width 0.4) (layer "F.Cu") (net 15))
 (segment (start 153.0215 71.224) (end 164 71.224) (width 0.4) (layer "F.Cu") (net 15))
 (segment (start 178 68) (end 188 68) (width 0.4) (layer "F.Cu") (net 15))
 (segment (start 164 71.224) (end 163.75895 71.224) (width 0.4) (layer "F.Cu") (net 15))
 (segment (start 153 98.01705) (end 153 76.7545) (width 0.4) (layer "F.Cu") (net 15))
 (segment (start 151.6465 75.401) (end 151.6465 72.599) (width 0.4) (layer "F.Cu") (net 15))
 (segment (start 188.97 68.97) (end 188.97 71.19) (width 0.4) (layer "F.Cu") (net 15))
 (segment (start 154.439 81.45605) (end 156.48295 83.5) (width 0.4) (layer "F.Cu") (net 15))
 (segment (start 151.6465 72.599) (end 153.0215 71.224) (width 0.4) (layer "F.Cu") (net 15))
 (segment (start 192.001 102.999) (end 194.583372 102.999) (width 0.4) (layer "B.Cu") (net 15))
 (segment (start 189.999 102.999) (end 189.999 87.461) (width 0.4) (layer "B.Cu") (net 15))
 (segment (start 197.499 105.001) (end 198.5 104) (width 0.4) (layer "B.Cu") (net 15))
 (segment (start 191 104) (end 192.001 102.999) (width 0.4) (layer "B.Cu") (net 15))
 (segment (start 189.999 87.461) (end 191.46 86) (width 0.4) (layer "B.Cu") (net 15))
 (segment (start 196.585372 105.001) (end 197.499 105.001) (width 0.4) (layer "B.Cu") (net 15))
 (segment (start 191 104) (end 189.999 102.999) (width 0.4) (layer "B.Cu") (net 15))
 (segment (start 194.583372 102.999) (end 196.585372 105.001) (width 0.4) (layer "B.Cu") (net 15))
 (segment (start 192.5 95) (end 191.5 96) (width 0.4) (layer "F.Cu") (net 6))
 (segment (start 173.625 74.525) (end 167.325 74.525) (width 0.4) (layer "F.Cu") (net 6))
 (segment (start 188 95) (end 188 90.55758) (width 0.4) (layer "F.Cu") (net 6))
 (segment (start 175.126 77.68358) (end 175.126 76.026) (width 0.4) (layer "F.Cu") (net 6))
 (segment (start 191.5 96) (end 189 96) (width 0.4) (layer "F.Cu") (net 6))
 (segment (start 189 96) (end 188 95) (width 0.4) (layer "F.Cu") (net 6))
 (segment (start 175.126 76.026) (end 173.625 74.525) (width 0.4) (layer "F.Cu") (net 6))
 (segment (start 188 90.55758) (end 175.126 77.68358) (width 0.4) (layer "F.Cu") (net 6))
 (segment (start 152.46 79) (end 150.46 81) (width 0.4) (layer "B.Cu") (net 34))
 (segment (start 196.249 71.749) (end 200 75.5) (width 0.4) (layer "B.Cu") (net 34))
 (segment (start 199 107) (end 186.68842 107) (width 0.4) (layer "B.Cu") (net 34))
 (segment (start 182.321819 72.481819) (end 193.599 72.481819) (width 0.4) (layer "B.Cu") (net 34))
 (segment (start 183.31158 107) (end 183.2 107) (width 0.4) (layer "B.Cu") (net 34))
 (segment (start 184.21258 104.099) (end 183.099 105.21258) (width 0.4) (layer "B.Cu") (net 34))
 (segment (start 183.2 107) (end 155.2 79) (width 0.4) (layer "B.Cu") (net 34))
 (segment (start 183.099 105.21258) (end 183.099 106.78742) (width 0.4) (layer "B.Cu") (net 34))
 (segment (start 193.599 72.481819) (end 194.331819 71.749) (width 0.4) (layer "B.Cu") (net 34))
 (segment (start 186.901 106.78742) (end 186.901 105.21258) (width 0.4) (layer "B.Cu") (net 34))
 (segment (start 194.331819 71.749) (end 196.249 71.749) (width 0.4) (layer "B.Cu") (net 34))
 (segment (start 183.099 106.78742) (end 183.31158 107) (width 0.4) (layer "B.Cu") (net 34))
 (segment (start 200 106) (end 199 107) (width 0.4) (layer "B.Cu") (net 34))
 (segment (start 200 75.5) (end 200 106) (width 0.4) (layer "B.Cu") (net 34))
 (segment (start 186.901 105.21258) (end 185.78742 104.099) (width 0.4) (layer "B.Cu") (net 34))
 (segment (start 186.68842 107) (end 186.901 106.78742) (width 0.4) (layer "B.Cu") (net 34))
 (segment (start 185.78742 104.099) (end 184.21258 104.099) (width 0.4) (layer "B.Cu") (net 34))
 (segment (start 155.2 79) (end 152.46 79) (width 0.4) (layer "B.Cu") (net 34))
 (segment (start 181.03 71.19) (end 182.321819 72.481819) (width 0.4) (layer "B.Cu") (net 34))
 (segment (start 180.064 72.764) (end 181.03 73.73) (width 0.4) (layer "B.Cu") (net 35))
 (segment (start 198.948942 107.901) (end 200.601 106.248942) (width 0.4) (layer "B.Cu") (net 35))
 (segment (start 200.601 106.248942) (end 200.601 72.401) (width 0.4) (layer "B.Cu") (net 35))
 (segment (start 180.064 70.224) (end 180.064 72.764) (width 0.4) (layer "B.Cu") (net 35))
 (segment (start 155.54 81) (end 182.441 107.901) (width 0.4) (layer "B.Cu") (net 35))
 (segment (start 182.441 107.901) (end 198.948942 107.901) (width 0.4) (layer "B.Cu") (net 35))
 (segment (start 200.601 72.401) (end 198.424 70.224) (width 0.4) (layer "B.Cu") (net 35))
 (segment (start 155.54 81) (end 155.54 87) (width 0.4) (layer "B.Cu") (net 35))
 (segment (start 198.424 70.224) (end 180.064 70.224) (width 0.4) (layer "B.Cu") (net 35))
 (segment (start 177.81 87.19) (end 172 93) (width 0.4) (layer "F.Cu") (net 31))
 (segment (start 172 93) (end 155.54 93) (width 0.4) (layer "F.Cu") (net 31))
 (segment (start 177.81 83.5) (end 177.81 87.19) (width 0.4) (layer "F.Cu") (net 31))
 (segment (start 150.46 93) (end 145.821 88.361) (width 0.4) (layer "F.Cu") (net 30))
 (segment (start 145.821 76.581) (end 144.62 75.38) (width 0.4) (layer "F.Cu") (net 30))
 (segment (start 145.821 88.361) (end 145.821 76.581) (width 0.4) (layer "F.Cu") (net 30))
 (segment (start 168.201 91.899) (end 155.08395 91.899) (width 0.4) (layer "F.Cu") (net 2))
 (segment (start 155.08395 91.899) (end 154.439 92.54395) (width 0.4) (layer "F.Cu") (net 2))
 (segment (start 154.439 97.899) (end 155.54 99) (width 0.4) (layer "F.Cu") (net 2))
 (segment (start 175.27 83.5) (end 175.27 84.83) (width 0.4) (layer "F.Cu") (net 2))
 (segment (start 175.27 84.83) (end 168.201 91.899) (width 0.4) (layer "F.Cu") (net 2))
 (segment (start 154.439 92.54395) (end 154.439 97.899) (width 0.4) (layer "F.Cu") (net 2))
 (segment (start 150.46 99) (end 151.561 97.899) (width 0.4) (layer "F.Cu") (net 1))
 (segment (start 151.561 79.781) (end 144.62 72.84) (width 0.4) (layer "F.Cu") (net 1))
 (segment (start 151.561 97.899) (end 151.561 79.781) (width 0.4) (layer "F.Cu") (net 1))
 (segment (start 191.537 88) (end 190 88) (width 0.4) (layer "F.Cu") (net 33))
 (segment (start 192.73 86) (end 192.73 86.807) (width 0.4) (layer "F.Cu") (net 33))
 (segment (start 192.73 86.807) (end 191.537 88) (width 0.4) (layer "F.Cu") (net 33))
 (segment (start 190 85.24) (end 181.03 76.27) (width 0.4) (layer "F.Cu") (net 33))
 (segment (start 190 88) (end 190 85.24) (width 0.4) (layer "F.Cu") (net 33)))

